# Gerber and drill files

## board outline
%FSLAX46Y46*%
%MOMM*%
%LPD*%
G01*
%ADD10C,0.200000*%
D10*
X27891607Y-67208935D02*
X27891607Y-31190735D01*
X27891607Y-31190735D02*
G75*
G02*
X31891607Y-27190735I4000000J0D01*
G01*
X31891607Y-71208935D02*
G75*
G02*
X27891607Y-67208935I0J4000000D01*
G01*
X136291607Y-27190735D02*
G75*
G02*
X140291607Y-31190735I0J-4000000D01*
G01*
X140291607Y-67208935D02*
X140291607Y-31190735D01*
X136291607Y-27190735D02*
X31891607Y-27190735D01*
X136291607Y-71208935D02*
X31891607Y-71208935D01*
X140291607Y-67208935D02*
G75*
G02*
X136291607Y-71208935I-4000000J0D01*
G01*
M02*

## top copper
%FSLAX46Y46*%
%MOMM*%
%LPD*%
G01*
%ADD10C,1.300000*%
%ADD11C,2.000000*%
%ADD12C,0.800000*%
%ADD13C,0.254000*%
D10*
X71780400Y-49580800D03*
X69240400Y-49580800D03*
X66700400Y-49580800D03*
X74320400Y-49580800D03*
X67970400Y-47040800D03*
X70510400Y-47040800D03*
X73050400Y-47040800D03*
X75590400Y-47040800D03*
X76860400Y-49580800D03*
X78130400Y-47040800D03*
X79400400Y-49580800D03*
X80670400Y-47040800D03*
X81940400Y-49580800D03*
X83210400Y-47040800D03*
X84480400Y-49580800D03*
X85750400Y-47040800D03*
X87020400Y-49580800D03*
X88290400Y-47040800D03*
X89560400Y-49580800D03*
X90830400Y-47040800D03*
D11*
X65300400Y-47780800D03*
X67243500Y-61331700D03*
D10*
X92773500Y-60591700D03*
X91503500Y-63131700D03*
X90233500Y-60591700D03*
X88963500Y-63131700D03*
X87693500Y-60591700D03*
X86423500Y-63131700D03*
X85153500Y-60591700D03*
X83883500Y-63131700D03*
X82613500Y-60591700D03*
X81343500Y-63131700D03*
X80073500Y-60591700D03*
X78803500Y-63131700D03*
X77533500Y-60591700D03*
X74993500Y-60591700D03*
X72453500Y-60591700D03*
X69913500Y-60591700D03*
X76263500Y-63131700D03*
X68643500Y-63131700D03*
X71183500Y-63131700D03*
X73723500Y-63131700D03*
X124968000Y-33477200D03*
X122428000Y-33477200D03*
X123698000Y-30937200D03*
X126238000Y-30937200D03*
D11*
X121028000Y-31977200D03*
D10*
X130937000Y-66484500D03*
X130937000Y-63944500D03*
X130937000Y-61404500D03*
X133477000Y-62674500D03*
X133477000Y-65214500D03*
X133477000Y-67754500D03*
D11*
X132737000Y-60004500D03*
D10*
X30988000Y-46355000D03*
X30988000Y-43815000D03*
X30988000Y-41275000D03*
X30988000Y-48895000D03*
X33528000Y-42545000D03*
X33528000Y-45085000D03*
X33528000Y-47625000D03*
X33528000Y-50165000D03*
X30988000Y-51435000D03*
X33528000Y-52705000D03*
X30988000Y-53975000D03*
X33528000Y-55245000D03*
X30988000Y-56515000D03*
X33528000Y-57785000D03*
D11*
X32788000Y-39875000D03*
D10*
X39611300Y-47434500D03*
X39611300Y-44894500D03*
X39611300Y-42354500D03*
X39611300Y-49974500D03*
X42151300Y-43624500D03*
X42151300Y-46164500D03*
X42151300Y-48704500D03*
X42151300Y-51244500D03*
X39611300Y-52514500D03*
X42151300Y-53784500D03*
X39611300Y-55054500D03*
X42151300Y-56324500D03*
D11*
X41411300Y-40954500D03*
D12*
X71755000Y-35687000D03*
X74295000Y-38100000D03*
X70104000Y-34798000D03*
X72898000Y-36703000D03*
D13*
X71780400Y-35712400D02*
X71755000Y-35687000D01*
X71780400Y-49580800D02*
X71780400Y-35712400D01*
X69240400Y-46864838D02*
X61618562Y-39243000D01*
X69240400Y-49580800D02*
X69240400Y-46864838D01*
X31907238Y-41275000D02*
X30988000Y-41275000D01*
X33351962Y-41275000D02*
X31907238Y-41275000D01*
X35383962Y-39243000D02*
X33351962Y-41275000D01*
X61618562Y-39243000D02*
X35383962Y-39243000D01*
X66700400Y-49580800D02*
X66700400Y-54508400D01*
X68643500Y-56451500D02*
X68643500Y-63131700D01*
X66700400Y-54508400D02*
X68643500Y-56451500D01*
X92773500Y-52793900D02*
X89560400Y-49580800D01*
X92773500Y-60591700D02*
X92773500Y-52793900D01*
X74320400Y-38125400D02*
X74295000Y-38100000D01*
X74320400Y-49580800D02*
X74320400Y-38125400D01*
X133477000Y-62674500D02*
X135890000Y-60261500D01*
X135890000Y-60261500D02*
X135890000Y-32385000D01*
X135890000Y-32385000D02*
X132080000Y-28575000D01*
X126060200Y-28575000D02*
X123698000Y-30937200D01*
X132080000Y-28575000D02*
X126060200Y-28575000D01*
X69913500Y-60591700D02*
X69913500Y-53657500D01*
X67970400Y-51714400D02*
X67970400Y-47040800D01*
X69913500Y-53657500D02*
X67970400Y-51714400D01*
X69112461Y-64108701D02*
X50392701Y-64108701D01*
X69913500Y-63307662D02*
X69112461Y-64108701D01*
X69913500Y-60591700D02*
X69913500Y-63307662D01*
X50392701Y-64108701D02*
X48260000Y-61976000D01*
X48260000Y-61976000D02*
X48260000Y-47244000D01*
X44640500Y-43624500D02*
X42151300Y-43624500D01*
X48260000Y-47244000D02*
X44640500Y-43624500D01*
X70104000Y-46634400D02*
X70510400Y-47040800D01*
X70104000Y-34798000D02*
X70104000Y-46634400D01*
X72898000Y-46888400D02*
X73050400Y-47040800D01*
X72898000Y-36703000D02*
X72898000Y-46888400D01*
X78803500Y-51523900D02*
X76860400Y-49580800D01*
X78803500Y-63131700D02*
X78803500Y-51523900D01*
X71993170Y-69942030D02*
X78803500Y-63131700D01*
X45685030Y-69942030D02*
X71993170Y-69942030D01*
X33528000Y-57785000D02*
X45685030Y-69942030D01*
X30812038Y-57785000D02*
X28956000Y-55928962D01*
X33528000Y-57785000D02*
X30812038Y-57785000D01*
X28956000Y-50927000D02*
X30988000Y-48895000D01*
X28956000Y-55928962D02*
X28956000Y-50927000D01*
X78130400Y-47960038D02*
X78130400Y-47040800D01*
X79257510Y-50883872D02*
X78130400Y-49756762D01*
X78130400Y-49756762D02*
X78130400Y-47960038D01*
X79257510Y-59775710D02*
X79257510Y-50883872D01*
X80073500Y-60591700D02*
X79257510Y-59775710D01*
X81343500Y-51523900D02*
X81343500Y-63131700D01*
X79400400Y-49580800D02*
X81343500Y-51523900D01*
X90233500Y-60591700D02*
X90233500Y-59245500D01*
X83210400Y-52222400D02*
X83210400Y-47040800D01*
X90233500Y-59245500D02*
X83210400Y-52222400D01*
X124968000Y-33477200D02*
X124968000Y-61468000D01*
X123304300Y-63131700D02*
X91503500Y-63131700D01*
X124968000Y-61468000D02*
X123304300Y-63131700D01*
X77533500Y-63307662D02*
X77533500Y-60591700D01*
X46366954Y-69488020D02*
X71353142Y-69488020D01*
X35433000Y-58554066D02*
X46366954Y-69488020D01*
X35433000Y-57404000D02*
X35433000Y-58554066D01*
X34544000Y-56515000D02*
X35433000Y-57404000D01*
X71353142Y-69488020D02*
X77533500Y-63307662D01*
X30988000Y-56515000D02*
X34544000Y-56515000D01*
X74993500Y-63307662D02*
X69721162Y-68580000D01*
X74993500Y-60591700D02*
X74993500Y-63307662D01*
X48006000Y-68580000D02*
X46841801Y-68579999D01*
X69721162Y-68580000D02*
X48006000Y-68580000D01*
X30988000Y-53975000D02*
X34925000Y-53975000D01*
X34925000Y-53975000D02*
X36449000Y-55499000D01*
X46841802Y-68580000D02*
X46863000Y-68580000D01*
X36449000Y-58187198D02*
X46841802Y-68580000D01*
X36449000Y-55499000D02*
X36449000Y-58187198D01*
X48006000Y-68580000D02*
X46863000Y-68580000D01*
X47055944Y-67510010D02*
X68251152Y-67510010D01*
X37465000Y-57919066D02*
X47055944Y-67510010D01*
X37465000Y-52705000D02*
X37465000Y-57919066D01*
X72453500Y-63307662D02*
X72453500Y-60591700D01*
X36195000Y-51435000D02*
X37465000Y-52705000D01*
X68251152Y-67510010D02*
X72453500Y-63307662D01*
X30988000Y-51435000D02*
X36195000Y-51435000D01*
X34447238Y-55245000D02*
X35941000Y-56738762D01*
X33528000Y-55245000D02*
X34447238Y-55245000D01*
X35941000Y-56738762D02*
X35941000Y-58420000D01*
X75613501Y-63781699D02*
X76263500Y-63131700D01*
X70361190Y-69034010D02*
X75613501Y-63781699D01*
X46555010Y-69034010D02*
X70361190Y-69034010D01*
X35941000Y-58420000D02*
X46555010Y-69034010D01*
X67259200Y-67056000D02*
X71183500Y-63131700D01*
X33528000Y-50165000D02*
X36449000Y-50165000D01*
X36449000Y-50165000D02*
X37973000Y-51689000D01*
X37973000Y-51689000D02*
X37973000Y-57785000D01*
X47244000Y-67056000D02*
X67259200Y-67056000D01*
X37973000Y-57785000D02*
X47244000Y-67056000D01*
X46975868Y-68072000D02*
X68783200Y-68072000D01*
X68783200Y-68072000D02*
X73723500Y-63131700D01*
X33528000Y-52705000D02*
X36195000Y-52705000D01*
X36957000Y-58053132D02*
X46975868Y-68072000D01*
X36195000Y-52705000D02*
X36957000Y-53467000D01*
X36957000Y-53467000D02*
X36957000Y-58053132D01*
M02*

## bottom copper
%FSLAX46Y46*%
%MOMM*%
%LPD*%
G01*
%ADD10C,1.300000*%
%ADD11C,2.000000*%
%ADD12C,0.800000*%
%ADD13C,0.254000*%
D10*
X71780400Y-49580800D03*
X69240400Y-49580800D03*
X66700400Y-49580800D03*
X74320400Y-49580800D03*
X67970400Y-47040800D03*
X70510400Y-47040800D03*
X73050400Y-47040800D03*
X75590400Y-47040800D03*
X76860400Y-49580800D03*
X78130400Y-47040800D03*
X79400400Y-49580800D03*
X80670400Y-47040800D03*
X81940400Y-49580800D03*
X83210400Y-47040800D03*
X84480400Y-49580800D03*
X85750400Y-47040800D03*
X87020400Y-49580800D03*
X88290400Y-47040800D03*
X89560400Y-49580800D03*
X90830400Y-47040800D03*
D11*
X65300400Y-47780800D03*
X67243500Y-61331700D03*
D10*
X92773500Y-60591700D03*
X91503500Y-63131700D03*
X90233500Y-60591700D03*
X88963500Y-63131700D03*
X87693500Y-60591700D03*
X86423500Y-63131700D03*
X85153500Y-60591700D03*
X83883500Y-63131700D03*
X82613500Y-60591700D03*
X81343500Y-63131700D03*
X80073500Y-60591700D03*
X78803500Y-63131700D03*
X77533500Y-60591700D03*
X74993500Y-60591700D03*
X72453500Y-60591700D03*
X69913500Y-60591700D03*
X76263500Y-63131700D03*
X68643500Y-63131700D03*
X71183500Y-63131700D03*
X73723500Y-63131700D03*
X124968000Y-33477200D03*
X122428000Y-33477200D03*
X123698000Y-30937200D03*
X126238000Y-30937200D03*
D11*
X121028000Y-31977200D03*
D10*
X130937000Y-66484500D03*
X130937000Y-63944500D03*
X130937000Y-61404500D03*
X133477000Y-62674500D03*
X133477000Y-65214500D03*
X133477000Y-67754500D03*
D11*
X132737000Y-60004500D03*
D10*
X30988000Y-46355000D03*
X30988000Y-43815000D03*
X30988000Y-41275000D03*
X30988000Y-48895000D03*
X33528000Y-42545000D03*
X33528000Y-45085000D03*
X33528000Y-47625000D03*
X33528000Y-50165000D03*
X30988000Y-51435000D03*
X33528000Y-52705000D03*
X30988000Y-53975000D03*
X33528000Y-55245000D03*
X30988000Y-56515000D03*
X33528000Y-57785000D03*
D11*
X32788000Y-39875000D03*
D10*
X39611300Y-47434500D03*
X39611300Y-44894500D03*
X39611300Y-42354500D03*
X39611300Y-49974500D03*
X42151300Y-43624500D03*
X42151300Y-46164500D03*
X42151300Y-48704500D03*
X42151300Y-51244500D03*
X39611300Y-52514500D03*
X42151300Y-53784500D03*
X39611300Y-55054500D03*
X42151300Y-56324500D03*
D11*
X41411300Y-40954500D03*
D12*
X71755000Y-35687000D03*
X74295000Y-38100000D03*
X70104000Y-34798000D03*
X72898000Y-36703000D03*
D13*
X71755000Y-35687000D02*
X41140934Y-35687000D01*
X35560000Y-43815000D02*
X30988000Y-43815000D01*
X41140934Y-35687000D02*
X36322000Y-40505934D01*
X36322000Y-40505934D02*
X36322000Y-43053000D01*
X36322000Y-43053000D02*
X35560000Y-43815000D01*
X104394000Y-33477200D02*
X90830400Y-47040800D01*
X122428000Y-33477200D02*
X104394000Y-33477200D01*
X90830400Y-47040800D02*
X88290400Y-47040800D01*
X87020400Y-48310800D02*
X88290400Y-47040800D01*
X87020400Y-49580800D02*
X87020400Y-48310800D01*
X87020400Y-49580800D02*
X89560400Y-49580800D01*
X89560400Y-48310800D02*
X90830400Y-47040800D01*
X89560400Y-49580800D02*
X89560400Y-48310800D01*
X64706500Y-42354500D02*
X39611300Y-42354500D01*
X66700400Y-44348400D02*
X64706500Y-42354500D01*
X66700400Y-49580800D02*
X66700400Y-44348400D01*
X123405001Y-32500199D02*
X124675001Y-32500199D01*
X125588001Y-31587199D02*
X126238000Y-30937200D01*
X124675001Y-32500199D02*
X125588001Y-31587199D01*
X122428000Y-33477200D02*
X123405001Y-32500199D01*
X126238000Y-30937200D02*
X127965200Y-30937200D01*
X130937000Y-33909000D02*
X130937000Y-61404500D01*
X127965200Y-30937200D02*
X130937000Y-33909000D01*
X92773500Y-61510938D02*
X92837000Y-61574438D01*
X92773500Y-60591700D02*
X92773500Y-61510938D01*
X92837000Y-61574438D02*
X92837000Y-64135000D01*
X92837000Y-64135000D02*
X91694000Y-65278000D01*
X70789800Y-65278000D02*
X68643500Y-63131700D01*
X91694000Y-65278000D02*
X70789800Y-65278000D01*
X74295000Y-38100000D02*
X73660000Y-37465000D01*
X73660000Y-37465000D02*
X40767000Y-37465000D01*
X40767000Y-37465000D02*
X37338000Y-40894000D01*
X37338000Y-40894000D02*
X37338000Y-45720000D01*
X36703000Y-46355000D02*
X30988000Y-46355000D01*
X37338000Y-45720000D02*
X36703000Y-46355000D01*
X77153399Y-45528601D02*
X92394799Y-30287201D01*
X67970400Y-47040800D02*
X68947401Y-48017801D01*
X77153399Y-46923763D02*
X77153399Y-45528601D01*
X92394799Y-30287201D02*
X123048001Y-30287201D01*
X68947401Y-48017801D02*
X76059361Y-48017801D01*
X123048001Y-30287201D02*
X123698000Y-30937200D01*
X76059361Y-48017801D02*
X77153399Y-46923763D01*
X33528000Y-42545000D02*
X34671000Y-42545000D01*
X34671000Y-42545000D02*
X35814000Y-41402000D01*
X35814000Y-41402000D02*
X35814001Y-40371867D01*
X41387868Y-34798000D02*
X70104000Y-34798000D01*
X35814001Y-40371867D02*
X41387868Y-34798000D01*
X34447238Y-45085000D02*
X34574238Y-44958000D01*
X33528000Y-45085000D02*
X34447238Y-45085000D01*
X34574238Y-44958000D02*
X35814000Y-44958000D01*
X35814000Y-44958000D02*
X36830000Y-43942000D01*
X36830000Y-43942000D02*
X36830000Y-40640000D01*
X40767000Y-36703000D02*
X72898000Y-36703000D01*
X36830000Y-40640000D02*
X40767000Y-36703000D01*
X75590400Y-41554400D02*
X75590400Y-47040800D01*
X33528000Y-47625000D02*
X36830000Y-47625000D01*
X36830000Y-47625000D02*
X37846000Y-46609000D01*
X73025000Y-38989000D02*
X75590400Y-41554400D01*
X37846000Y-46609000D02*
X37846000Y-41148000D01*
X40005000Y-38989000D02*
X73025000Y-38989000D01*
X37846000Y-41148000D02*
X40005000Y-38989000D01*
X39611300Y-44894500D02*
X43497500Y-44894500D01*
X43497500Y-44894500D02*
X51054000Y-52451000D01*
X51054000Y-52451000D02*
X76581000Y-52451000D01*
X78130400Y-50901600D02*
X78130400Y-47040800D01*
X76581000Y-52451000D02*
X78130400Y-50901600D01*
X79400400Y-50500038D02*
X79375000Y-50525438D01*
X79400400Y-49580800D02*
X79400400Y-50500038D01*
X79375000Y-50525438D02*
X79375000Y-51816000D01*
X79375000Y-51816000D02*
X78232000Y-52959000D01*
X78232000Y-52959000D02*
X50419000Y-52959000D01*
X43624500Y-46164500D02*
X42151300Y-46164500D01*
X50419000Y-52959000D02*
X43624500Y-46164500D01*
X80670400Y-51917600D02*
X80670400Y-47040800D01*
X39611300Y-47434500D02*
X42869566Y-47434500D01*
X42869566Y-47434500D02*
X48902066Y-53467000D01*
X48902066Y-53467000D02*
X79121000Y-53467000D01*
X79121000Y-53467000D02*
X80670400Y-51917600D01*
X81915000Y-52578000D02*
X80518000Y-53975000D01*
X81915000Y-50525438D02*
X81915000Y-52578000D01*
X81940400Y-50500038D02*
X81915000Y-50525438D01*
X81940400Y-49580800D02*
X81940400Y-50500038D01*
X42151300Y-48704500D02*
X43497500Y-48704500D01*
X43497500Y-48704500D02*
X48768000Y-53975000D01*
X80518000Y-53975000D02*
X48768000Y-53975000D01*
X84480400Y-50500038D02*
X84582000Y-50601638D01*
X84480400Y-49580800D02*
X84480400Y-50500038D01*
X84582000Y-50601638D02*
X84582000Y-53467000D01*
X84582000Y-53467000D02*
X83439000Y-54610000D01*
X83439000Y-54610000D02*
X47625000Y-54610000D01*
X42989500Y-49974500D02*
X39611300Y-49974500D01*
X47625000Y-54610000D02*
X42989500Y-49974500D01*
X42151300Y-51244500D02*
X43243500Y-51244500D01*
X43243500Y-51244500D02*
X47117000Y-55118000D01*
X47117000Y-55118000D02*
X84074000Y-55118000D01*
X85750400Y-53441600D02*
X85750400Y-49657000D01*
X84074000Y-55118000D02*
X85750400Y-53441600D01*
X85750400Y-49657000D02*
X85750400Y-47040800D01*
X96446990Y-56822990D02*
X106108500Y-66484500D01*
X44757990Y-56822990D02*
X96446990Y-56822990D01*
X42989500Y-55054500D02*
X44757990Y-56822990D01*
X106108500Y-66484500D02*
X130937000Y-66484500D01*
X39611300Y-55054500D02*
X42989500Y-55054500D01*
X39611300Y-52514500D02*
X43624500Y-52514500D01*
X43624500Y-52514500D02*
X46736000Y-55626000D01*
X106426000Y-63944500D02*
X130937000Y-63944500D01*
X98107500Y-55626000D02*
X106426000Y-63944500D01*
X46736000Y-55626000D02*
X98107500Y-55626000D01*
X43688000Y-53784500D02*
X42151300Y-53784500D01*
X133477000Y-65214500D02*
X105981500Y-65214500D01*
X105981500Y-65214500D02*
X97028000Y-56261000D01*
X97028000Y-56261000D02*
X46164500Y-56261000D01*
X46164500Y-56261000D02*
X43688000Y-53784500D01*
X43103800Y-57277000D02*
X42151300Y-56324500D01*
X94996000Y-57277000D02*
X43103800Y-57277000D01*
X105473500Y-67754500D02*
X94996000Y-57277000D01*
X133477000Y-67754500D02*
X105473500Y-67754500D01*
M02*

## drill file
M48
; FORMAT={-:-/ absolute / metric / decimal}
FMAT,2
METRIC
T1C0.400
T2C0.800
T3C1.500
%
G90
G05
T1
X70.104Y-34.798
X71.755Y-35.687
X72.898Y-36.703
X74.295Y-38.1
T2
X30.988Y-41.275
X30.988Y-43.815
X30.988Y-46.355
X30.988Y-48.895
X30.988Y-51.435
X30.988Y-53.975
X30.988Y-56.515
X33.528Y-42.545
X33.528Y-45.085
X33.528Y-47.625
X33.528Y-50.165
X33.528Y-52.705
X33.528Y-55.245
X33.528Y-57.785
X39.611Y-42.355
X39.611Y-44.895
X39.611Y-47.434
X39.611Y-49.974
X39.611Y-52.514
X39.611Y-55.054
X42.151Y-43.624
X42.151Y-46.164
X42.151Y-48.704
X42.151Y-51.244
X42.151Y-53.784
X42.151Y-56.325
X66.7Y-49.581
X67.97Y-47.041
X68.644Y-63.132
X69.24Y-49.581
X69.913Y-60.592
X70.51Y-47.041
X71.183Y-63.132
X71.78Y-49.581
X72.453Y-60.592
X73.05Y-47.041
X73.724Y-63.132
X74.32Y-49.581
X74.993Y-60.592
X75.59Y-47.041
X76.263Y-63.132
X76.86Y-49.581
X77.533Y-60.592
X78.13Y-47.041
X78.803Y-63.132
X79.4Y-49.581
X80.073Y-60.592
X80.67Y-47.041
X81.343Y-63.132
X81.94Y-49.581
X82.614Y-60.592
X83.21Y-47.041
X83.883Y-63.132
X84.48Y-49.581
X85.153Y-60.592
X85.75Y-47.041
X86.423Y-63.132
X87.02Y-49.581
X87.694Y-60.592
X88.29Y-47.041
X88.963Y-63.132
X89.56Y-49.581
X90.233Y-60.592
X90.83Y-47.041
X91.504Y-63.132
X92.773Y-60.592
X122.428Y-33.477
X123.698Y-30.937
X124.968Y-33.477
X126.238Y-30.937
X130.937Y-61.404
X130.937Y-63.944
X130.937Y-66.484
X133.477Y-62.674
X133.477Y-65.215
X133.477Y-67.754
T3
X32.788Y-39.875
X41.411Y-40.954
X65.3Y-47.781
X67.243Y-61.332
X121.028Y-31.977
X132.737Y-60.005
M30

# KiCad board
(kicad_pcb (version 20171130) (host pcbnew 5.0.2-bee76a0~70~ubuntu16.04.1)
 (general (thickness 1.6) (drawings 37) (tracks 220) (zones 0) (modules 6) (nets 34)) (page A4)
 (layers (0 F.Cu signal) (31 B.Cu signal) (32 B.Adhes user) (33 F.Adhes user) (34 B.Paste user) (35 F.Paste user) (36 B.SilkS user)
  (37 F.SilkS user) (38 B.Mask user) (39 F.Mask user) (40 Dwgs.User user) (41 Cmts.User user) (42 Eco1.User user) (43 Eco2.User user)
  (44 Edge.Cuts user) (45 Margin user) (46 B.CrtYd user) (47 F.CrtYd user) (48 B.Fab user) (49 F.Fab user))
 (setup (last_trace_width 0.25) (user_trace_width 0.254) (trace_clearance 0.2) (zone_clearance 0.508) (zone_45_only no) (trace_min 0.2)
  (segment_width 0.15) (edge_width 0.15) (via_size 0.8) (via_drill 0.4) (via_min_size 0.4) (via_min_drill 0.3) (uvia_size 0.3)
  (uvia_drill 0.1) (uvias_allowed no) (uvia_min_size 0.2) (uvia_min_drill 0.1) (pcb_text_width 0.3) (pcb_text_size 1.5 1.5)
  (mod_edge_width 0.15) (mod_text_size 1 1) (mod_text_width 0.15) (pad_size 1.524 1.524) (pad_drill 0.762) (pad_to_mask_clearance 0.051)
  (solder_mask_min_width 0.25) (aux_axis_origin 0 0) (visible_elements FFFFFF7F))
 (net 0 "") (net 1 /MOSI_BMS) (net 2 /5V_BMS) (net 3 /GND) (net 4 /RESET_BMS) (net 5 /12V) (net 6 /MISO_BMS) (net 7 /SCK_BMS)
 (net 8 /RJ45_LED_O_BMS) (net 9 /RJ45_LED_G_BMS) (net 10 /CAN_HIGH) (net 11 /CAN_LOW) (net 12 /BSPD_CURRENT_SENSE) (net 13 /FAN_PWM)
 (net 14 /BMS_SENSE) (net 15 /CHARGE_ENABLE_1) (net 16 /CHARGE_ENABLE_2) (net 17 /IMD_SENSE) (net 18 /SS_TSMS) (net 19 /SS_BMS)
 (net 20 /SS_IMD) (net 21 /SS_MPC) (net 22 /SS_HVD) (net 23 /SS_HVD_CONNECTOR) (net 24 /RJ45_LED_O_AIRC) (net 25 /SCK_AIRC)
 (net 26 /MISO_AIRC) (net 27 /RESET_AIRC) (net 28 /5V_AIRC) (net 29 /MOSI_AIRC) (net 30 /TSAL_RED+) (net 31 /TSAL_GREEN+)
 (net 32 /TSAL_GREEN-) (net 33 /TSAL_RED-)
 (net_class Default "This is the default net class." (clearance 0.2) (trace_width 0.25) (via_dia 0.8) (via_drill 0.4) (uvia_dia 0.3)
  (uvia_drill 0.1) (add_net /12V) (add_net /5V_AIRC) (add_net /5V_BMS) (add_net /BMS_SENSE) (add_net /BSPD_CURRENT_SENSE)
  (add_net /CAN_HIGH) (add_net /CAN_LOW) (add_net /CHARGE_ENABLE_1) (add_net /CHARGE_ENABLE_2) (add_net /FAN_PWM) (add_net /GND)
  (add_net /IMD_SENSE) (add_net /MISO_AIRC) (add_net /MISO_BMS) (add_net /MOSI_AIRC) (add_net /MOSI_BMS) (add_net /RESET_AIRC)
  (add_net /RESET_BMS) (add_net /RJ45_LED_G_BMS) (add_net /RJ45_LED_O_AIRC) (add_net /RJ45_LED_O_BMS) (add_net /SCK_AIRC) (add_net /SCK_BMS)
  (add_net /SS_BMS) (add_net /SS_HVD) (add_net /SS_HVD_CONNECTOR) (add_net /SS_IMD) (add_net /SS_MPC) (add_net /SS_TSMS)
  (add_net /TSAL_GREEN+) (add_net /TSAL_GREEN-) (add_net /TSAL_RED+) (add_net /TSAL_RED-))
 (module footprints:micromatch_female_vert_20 (layer F.Cu) (at 71.7804 49.5808 90)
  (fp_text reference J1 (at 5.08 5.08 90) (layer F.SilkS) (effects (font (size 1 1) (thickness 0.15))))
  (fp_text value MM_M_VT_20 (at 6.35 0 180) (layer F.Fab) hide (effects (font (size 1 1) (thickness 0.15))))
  (pad 5 thru_hole circle (at 0 0 90) (size 1.3 1.3) (drill 0.8) (layers *.Cu *.Mask) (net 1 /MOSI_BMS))
  (pad 3 thru_hole circle (at 0 -2.54 90) (size 1.3 1.3) (drill 0.8) (layers *.Cu *.Mask) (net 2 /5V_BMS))
  (pad 1 thru_hole circle (at 0 -5.08 90) (size 1.3 1.3) (drill 0.8) (layers *.Cu *.Mask) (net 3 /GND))
  (pad 7 thru_hole circle (at 0 2.54 90) (size 1.3 1.3) (drill 0.8) (layers *.Cu *.Mask) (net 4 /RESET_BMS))
  (pad 2 thru_hole circle (at 2.54 -3.81 90) (size 1.3 1.3) (drill 0.8) (layers *.Cu *.Mask) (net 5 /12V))
  (pad 4 thru_hole circle (at 2.54 -1.27 90) (size 1.3 1.3) (drill 0.8) (layers *.Cu *.Mask) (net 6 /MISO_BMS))
  (pad 6 thru_hole circle (at 2.54 1.27 90) (size 1.3 1.3) (drill 0.8) (layers *.Cu *.Mask) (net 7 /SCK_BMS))
  (pad 8 thru_hole circle (at 2.54 3.81 90) (size 1.3 1.3) (drill 0.8) (layers *.Cu *.Mask) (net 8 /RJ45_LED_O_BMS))
  (pad 9 thru_hole circle (at 0 5.08 90) (size 1.3 1.3) (drill 0.8) (layers *.Cu *.Mask) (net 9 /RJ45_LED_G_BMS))
  (pad 10 thru_hole circle (at 2.54 6.35 90) (size 1.3 1.3) (drill 0.8) (layers *.Cu *.Mask) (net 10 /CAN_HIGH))
  (pad 11 thru_hole circle (at 0 7.62 90) (size 1.3 1.3) (drill 0.8) (layers *.Cu *.Mask) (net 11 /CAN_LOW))
  (pad 12 thru_hole circle (at 2.54 8.89 90) (size 1.3 1.3) (drill 0.8) (layers *.Cu *.Mask) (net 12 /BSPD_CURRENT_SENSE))
  (pad 13 thru_hole circle (at 0 10.16 90) (size 1.3 1.3) (drill 0.8) (layers *.Cu *.Mask) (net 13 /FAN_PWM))
  (pad 14 thru_hole circle (at 2.54 11.43 90) (size 1.3 1.3) (drill 0.8) (layers *.Cu *.Mask) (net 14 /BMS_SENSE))
  (pad 15 thru_hole circle (at 0 12.7 90) (size 1.3 1.3) (drill 0.8) (layers *.Cu *.Mask) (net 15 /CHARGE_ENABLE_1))
  (pad 16 thru_hole circle (at 2.54 13.97 90) (size 1.3 1.3) (drill 0.8) (layers *.Cu *.Mask) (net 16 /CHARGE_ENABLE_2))
  (pad 17 thru_hole circle (at 0 15.24 90) (size 1.3 1.3) (drill 0.8) (layers *.Cu *.Mask) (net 3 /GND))
  (pad 18 thru_hole circle (at 2.54 16.51 90) (size 1.3 1.3) (drill 0.8) (layers *.Cu *.Mask) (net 3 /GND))
  (pad 19 thru_hole circle (at 0 17.78 90) (size 1.3 1.3) (drill 0.8) (layers *.Cu *.Mask) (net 3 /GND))
  (pad 20 thru_hole circle (at 2.54 19.05 90) (size 1.3 1.3) (drill 0.8) (layers *.Cu *.Mask) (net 3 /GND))
  (pad 21 thru_hole circle (at 1.8 -6.48 90) (size 2 2) (drill 1.5) (layers *.Cu *.Mask)))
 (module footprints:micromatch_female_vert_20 (layer F.Cu) (at 73.7235 63.1317 90)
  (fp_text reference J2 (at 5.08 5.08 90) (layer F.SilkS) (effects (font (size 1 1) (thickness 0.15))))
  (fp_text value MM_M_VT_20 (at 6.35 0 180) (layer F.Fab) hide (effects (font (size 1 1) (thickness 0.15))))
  (pad 21 thru_hole circle (at 1.8 -6.48 90) (size 2 2) (drill 1.5) (layers *.Cu *.Mask))
  (pad 20 thru_hole circle (at 2.54 19.05 90) (size 1.3 1.3) (drill 0.8) (layers *.Cu *.Mask) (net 3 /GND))
  (pad 19 thru_hole circle (at 0 17.78 90) (size 1.3 1.3) (drill 0.8) (layers *.Cu *.Mask) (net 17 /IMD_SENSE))
  (pad 18 thru_hole circle (at 2.54 16.51 90) (size 1.3 1.3) (drill 0.8) (layers *.Cu *.Mask) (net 14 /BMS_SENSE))
  (pad 17 thru_hole circle (at 0 15.24 90) (size 1.3 1.3) (drill 0.8) (layers *.Cu *.Mask) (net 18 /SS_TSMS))
  (pad 16 thru_hole circle (at 2.54 13.97 90) (size 1.3 1.3) (drill 0.8) (layers *.Cu *.Mask) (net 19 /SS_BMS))
  (pad 15 thru_hole circle (at 0 12.7 90) (size 1.3 1.3) (drill 0.8) (layers *.Cu *.Mask) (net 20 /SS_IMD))
  (pad 14 thru_hole circle (at 2.54 11.43 90) (size 1.3 1.3) (drill 0.8) (layers *.Cu *.Mask) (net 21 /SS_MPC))
  (pad 13 thru_hole circle (at 0 10.16 90) (size 1.3 1.3) (drill 0.8) (layers *.Cu *.Mask) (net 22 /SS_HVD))
  (pad 12 thru_hole circle (at 2.54 8.89 90) (size 1.3 1.3) (drill 0.8) (layers *.Cu *.Mask) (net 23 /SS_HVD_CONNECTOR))
  (pad 11 thru_hole circle (at 0 7.62 90) (size 1.3 1.3) (drill 0.8) (layers *.Cu *.Mask) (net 11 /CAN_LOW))
  (pad 10 thru_hole circle (at 2.54 6.35 90) (size 1.3 1.3) (drill 0.8) (layers *.Cu *.Mask) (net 10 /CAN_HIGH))
  (pad 9 thru_hole circle (at 0 5.08 90) (size 1.3 1.3) (drill 0.8) (layers *.Cu *.Mask) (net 9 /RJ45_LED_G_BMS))
  (pad 8 thru_hole circle (at 2.54 3.81 90) (size 1.3 1.3) (drill 0.8) (layers *.Cu *.Mask) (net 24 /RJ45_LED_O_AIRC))
  (pad 6 thru_hole circle (at 2.54 1.27 90) (size 1.3 1.3) (drill 0.8) (layers *.Cu *.Mask) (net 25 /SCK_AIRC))
  (pad 4 thru_hole circle (at 2.54 -1.27 90) (size 1.3 1.3) (drill 0.8) (layers *.Cu *.Mask) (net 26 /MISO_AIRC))
  (pad 2 thru_hole circle (at 2.54 -3.81 90) (size 1.3 1.3) (drill 0.8) (layers *.Cu *.Mask) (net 5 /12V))
  (pad 7 thru_hole circle (at 0 2.54 90) (size 1.3 1.3) (drill 0.8) (layers *.Cu *.Mask) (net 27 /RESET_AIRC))
  (pad 1 thru_hole circle (at 0 -5.08 90) (size 1.3 1.3) (drill 0.8) (layers *.Cu *.Mask) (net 3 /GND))
  (pad 3 thru_hole circle (at 0 -2.54 90) (size 1.3 1.3) (drill 0.8) (layers *.Cu *.Mask) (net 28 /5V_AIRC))
  (pad 5 thru_hole circle (at 0 0 90) (size 1.3 1.3) (drill 0.8) (layers *.Cu *.Mask) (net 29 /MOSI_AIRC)))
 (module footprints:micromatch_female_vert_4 (layer F.Cu) (at 127.508 33.4772 90)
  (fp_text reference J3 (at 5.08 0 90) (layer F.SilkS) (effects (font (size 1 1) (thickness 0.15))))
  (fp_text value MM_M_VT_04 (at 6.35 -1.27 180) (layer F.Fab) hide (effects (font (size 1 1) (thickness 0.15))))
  (pad 3 thru_hole circle (at 0 -2.54 90) (size 1.3 1.3) (drill 0.8) (layers *.Cu *.Mask) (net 17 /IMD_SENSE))
  (pad 1 thru_hole circle (at 0 -5.08 90) (size 1.3 1.3) (drill 0.8) (layers *.Cu *.Mask) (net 3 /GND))
  (pad 2 thru_hole circle (at 2.54 -3.81 90) (size 1.3 1.3) (drill 0.8) (layers *.Cu *.Mask) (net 5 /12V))
  (pad 4 thru_hole circle (at 2.54 -1.27 90) (size 1.3 1.3) (drill 0.8) (layers *.Cu *.Mask) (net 3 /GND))
  (pad 5 thru_hole circle (at 1.5 -6.48 90) (size 2 2) (drill 1.5) (layers *.Cu *.Mask)))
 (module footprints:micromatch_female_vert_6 (layer F.Cu) (at 130.937 66.4845)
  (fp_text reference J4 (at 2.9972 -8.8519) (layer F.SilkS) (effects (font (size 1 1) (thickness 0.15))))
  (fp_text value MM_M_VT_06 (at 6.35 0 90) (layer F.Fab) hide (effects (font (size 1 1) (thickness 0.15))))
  (pad 5 thru_hole circle (at 0 0) (size 1.3 1.3) (drill 0.8) (layers *.Cu *.Mask) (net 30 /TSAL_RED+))
  (pad 3 thru_hole circle (at 0 -2.54) (size 1.3 1.3) (drill 0.8) (layers *.Cu *.Mask) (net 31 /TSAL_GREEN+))
  (pad 1 thru_hole circle (at 0 -5.08) (size 1.3 1.3) (drill 0.8) (layers *.Cu *.Mask) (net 3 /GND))
  (pad 2 thru_hole circle (at 2.54 -3.81) (size 1.3 1.3) (drill 0.8) (layers *.Cu *.Mask) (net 5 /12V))
  (pad 4 thru_hole circle (at 2.54 -1.27) (size 1.3 1.3) (drill 0.8) (layers *.Cu *.Mask) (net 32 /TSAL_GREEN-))
  (pad 6 thru_hole circle (at 2.54 1.27) (size 1.3 1.3) (drill 0.8) (layers *.Cu *.Mask) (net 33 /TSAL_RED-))
  (pad 7 thru_hole circle (at 1.8 -6.48) (size 2 2) (drill 1.5) (layers *.Cu *.Mask)))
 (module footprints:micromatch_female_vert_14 (layer F.Cu) (at 30.988 46.355)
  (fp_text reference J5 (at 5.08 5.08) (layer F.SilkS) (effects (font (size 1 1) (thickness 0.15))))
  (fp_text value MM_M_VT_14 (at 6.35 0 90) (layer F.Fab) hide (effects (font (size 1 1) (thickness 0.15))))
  (pad 5 thru_hole circle (at 0 0) (size 1.3 1.3) (drill 0.8) (layers *.Cu *.Mask) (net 4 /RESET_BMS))
  (pad 3 thru_hole circle (at 0 -2.54) (size 1.3 1.3) (drill 0.8) (layers *.Cu *.Mask) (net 1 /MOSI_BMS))
  (pad 1 thru_hole circle (at 0 -5.08) (size 1.3 1.3) (drill 0.8) (layers *.Cu *.Mask) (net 2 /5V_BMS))
  (pad 7 thru_hole circle (at 0 2.54) (size 1.3 1.3) (drill 0.8) (layers *.Cu *.Mask) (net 9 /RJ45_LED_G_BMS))
  (pad 2 thru_hole circle (at 2.54 -3.81) (size 1.3 1.3) (drill 0.8) (layers *.Cu *.Mask) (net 6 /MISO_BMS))
  (pad 4 thru_hole circle (at 2.54 -1.27) (size 1.3 1.3) (drill 0.8) (layers *.Cu *.Mask) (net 7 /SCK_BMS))
  (pad 6 thru_hole circle (at 2.54 1.27) (size 1.3 1.3) (drill 0.8) (layers *.Cu *.Mask) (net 8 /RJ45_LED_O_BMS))
  (pad 8 thru_hole circle (at 2.54 3.81) (size 1.3 1.3) (drill 0.8) (layers *.Cu *.Mask) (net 28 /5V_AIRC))
  (pad 9 thru_hole circle (at 0 5.08) (size 1.3 1.3) (drill 0.8) (layers *.Cu *.Mask) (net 26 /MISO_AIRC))
  (pad 10 thru_hole circle (at 2.54 6.35) (size 1.3 1.3) (drill 0.8) (layers *.Cu *.Mask) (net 29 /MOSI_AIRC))
  (pad 11 thru_hole circle (at 0 7.62) (size 1.3 1.3) (drill 0.8) (layers *.Cu *.Mask) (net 25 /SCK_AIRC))
  (pad 12 thru_hole circle (at 2.54 8.89) (size 1.3 1.3) (drill 0.8) (layers *.Cu *.Mask) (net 27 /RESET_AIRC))
  (pad 13 thru_hole circle (at 0 10.16) (size 1.3 1.3) (drill 0.8) (layers *.Cu *.Mask) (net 24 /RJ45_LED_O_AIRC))
  (pad 14 thru_hole circle (at 2.54 11.43) (size 1.3 1.3) (drill 0.8) (layers *.Cu *.Mask) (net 9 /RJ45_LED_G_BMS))
  (pad 15 thru_hole circle (at 1.8 -6.48) (size 2 2) (drill 1.5) (layers *.Cu *.Mask)))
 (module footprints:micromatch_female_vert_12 (layer F.Cu) (at 39.6113 47.4345)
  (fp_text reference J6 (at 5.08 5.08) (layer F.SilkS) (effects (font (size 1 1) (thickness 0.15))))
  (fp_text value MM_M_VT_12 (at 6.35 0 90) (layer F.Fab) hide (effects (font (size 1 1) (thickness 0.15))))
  (pad 5 thru_hole circle (at 0 0) (size 1.3 1.3) (drill 0.8) (layers *.Cu *.Mask) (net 12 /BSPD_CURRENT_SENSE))
  (pad 3 thru_hole circle (at 0 -2.54) (size 1.3 1.3) (drill 0.8) (layers *.Cu *.Mask) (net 10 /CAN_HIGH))
  (pad 1 thru_hole circle (at 0 -5.08) (size 1.3 1.3) (drill 0.8) (layers *.Cu *.Mask) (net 3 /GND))
  (pad 7 thru_hole circle (at 0 2.54) (size 1.3 1.3) (drill 0.8) (layers *.Cu *.Mask) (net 15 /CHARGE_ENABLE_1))
  (pad 2 thru_hole circle (at 2.54 -3.81) (size 1.3 1.3) (drill 0.8) (layers *.Cu *.Mask) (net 5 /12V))
  (pad 4 thru_hole circle (at 2.54 -1.27) (size 1.3 1.3) (drill 0.8) (layers *.Cu *.Mask) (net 11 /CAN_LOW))
  (pad 6 thru_hole circle (at 2.54 1.27) (size 1.3 1.3) (drill 0.8) (layers *.Cu *.Mask) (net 13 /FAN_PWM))
  (pad 8 thru_hole circle (at 2.54 3.81) (size 1.3 1.3) (drill 0.8) (layers *.Cu *.Mask) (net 16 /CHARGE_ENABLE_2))
  (pad 9 thru_hole circle (at 0 5.08) (size 1.3 1.3) (drill 0.8) (layers *.Cu *.Mask) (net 31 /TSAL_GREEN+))
  (pad 10 thru_hole circle (at 2.54 6.35) (size 1.3 1.3) (drill 0.8) (layers *.Cu *.Mask) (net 32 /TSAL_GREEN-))
  (pad 11 thru_hole circle (at 0 7.62) (size 1.3 1.3) (drill 0.8) (layers *.Cu *.Mask) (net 30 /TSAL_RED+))
  (pad 12 thru_hole circle (at 2.54 8.89) (size 1.3 1.3) (drill 0.8) (layers *.Cu *.Mask) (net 33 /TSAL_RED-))
  (pad 13 thru_hole circle (at 1.8 -6.48) (size 2 2) (drill 1.5) (layers *.Cu *.Mask)))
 (gr_line (start 27.891607 67.208935) (end 27.891607 31.190735) (layer Edge.Cuts) (width 0.2))
 (gr_arc (start 31.891607 31.190735) (end 31.891607 27.190735) (angle -90) (layer Edge.Cuts) (width 0.2))
 (gr_arc (start 31.891607 67.208935) (end 27.891607 67.208935) (angle -90) (layer Edge.Cuts) (width 0.2))
 (gr_arc (start 136.291607 31.190735) (end 140.291607 31.190735) (angle -90) (layer Edge.Cuts) (width 0.2))
 (gr_line (start 140.291607 67.208935) (end 140.291607 31.190735) (layer Edge.Cuts) (width 0.2))
 (gr_line (start 136.291607 27.190735) (end 31.891607 27.190735) (layer Edge.Cuts) (width 0.2))
 (gr_line (start 136.291607 71.208935) (end 31.891607 71.208935) (layer Edge.Cuts) (width 0.2))
 (gr_arc (start 136.291607 67.208935) (end 136.291607 71.208935) (angle -90) (layer Edge.Cuts) (width 0.2))
 (via (at 71.755 35.687) (size 0.8) (drill 0.4) (layers F.Cu B.Cu) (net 1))
 (segment (start 71.7804 35.7124) (end 71.755 35.687) (width 0.254) (layer F.Cu) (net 1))
 (segment (start 71.7804 49.5808) (end 71.7804 35.7124) (width 0.254) (layer F.Cu) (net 1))
 (segment (start 71.755 35.687) (end 41.140934 35.687) (width 0.254) (layer B.Cu) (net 1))
 (segment (start 35.56 43.815) (end 30.988 43.815) (width 0.254) (layer B.Cu) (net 1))
 (segment (start 41.140934 35.687) (end 36.322 40.505934) (width 0.254) (layer B.Cu) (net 1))
 (segment (start 36.322 40.505934) (end 36.322 43.053) (width 0.254) (layer B.Cu) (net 1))
 (segment (start 36.322 43.053) (end 35.56 43.815) (width 0.254) (layer B.Cu) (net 1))
 (segment (start 69.2404 46.864838) (end 61.618562 39.243) (width 0.254) (layer F.Cu) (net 2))
 (segment (start 69.2404 49.5808) (end 69.2404 46.864838) (width 0.254) (layer F.Cu) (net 2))
 (segment (start 31.907238 41.275) (end 30.988 41.275) (width 0.254) (layer F.Cu) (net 2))
 (segment (start 33.351962 41.275) (end 31.907238 41.275) (width 0.254) (layer F.Cu) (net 2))
 (segment (start 35.383962 39.243) (end 33.351962 41.275) (width 0.254) (layer F.Cu) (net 2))
 (segment (start 61.618562 39.243) (end 35.383962 39.243) (width 0.254) (layer F.Cu) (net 2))
 (segment (start 104.394 33.4772) (end 90.8304 47.0408) (width 0.254) (layer B.Cu) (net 3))
 (segment (start 122.428 33.4772) (end 104.394 33.4772) (width 0.254) (layer B.Cu) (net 3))
 (segment (start 90.8304 47.0408) (end 88.2904 47.0408) (width 0.254) (layer B.Cu) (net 3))
 (segment (start 87.0204 48.3108) (end 88.2904 47.0408) (width 0.254) (layer B.Cu) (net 3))
 (segment (start 87.0204 49.5808) (end 87.0204 48.3108) (width 0.254) (layer B.Cu) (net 3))
 (segment (start 87.0204 49.5808) (end 89.5604 49.5808) (width 0.254) (layer B.Cu) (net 3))
 (segment (start 89.5604 48.3108) (end 90.8304 47.0408) (width 0.254) (layer B.Cu) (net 3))
 (segment (start 89.5604 49.5808) (end 89.5604 48.3108) (width 0.254) (layer B.Cu) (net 3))
 (segment (start 64.7065 42.3545) (end 39.6113 42.3545) (width 0.254) (layer B.Cu) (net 3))
 (segment (start 66.7004 44.3484) (end 64.7065 42.3545) (width 0.254) (layer B.Cu) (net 3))
 (segment (start 66.7004 49.5808) (end 66.7004 44.3484) (width 0.254) (layer B.Cu) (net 3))
 (segment (start 123.405001 32.500199) (end 124.675001 32.500199) (width 0.254) (layer B.Cu) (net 3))
 (segment (start 125.588001 31.587199) (end 126.238 30.9372) (width 0.254) (layer B.Cu) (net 3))
 (segment (start 124.675001 32.500199) (end 125.588001 31.587199) (width 0.254) (layer B.Cu) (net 3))
 (segment (start 122.428 33.4772) (end 123.405001 32.500199) (width 0.254) (layer B.Cu) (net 3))
 (segment (start 126.238 30.9372) (end 127.9652 30.9372) (width 0.254) (layer B.Cu) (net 3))
 (segment (start 130.937 33.909) (end 130.937 61.4045) (width 0.254) (layer B.Cu) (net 3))
 (segment (start 127.9652 30.9372) (end 130.937 33.909) (width 0.254) (layer B.Cu) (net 3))
 (segment (start 66.7004 49.5808) (end 66.7004 54.5084) (width 0.254) (layer F.Cu) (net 3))
 (segment (start 68.6435 56.4515) (end 68.6435 63.1317) (width 0.254) (layer F.Cu) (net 3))
 (segment (start 66.7004 54.5084) (end 68.6435 56.4515) (width 0.254) (layer F.Cu) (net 3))
 (segment (start 92.7735 52.7939) (end 89.5604 49.5808) (width 0.254) (layer F.Cu) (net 3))
 (segment (start 92.7735 60.5917) (end 92.7735 52.7939) (width 0.254) (layer F.Cu) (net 3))
 (segment (start 92.7735 61.510938) (end 92.837 61.574438) (width 0.254) (layer B.Cu) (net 3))
 (segment (start 92.7735 60.5917) (end 92.7735 61.510938) (width 0.254) (layer B.Cu) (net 3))
 (segment (start 92.837 61.574438) (end 92.837 64.135) (width 0.254) (layer B.Cu) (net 3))
 (segment (start 92.837 64.135) (end 91.694 65.278) (width 0.254) (layer B.Cu) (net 3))
 (segment (start 70.7898 65.278) (end 68.6435 63.1317) (width 0.254) (layer B.Cu) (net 3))
 (segment (start 91.694 65.278) (end 70.7898 65.278) (width 0.254) (layer B.Cu) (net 3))
 (via (at 74.295 38.1) (size 0.8) (drill 0.4) (layers F.Cu B.Cu) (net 4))
 (segment (start 74.3204 38.1254) (end 74.295 38.1) (width 0.254) (layer F.Cu) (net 4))
 (segment (start 74.3204 49.5808) (end 74.3204 38.1254) (width 0.254) (layer F.Cu) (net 4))
 (segment (start 74.295 38.1) (end 73.66 37.465) (width 0.254) (layer B.Cu) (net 4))
 (segment (start 73.66 37.465) (end 40.767 37.465) (width 0.254) (layer B.Cu) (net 4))
 (segment (start 40.767 37.465) (end 37.338 40.894) (width 0.254) (layer B.Cu) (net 4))
 (segment (start 37.338 40.894) (end 37.338 45.72) (width 0.254) (layer B.Cu) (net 4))
 (segment (start 36.703 46.355) (end 30.988 46.355) (width 0.254) (layer B.Cu) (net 4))
 (segment (start 37.338 45.72) (end 36.703 46.355) (width 0.254) (layer B.Cu) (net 4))
 (segment (start 133.477 62.6745) (end 135.89 60.2615) (width 0.254) (layer F.Cu) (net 5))
 (segment (start 135.89 60.2615) (end 135.89 32.385) (width 0.254) (layer F.Cu) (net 5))
 (segment (start 135.89 32.385) (end 132.08 28.575) (width 0.254) (layer F.Cu) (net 5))
 (segment (start 126.0602 28.575) (end 123.698 30.9372) (width 0.254) (layer F.Cu) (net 5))
 (segment (start 132.08 28.575) (end 126.0602 28.575) (width 0.254) (layer F.Cu) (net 5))
 (segment (start 69.9135 60.5917) (end 69.9135 53.6575) (width 0.254) (layer F.Cu) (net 5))
 (segment (start 67.9704 51.7144) (end 67.9704 47.0408) (width 0.254) (layer F.Cu) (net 5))
 (segment (start 69.9135 53.6575) (end 67.9704 51.7144) (width 0.254) (layer F.Cu) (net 5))
 (segment (start 69.112461 64.108701) (end 50.392701 64.108701) (width 0.254) (layer F.Cu) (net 5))
 (segment (start 69.9135 63.307662) (end 69.112461 64.108701) (width 0.254) (layer F.Cu) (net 5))
 (segment (start 69.9135 60.5917) (end 69.9135 63.307662) (width 0.254) (layer F.Cu) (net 5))
 (segment (start 50.392701 64.108701) (end 48.26 61.976) (width 0.254) (layer F.Cu) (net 5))
 (segment (start 48.26 61.976) (end 48.26 47.244) (width 0.254) (layer F.Cu) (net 5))
 (segment (start 44.6405 43.6245) (end 42.1513 43.6245) (width 0.254) (layer F.Cu) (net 5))
 (segment (start 48.26 47.244) (end 44.6405 43.6245) (width 0.254) (layer F.Cu) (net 5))
 (segment (start 77.153399 45.528601) (end 92.394799 30.287201) (width 0.254) (layer B.Cu) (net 5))
 (segment (start 67.9704 47.0408) (end 68.947401 48.017801) (width 0.254) (layer B.Cu) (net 5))
 (segment (start 77.153399 46.923763) (end 77.153399 45.528601) (width 0.254) (layer B.Cu) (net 5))
 (segment (start 92.394799 30.287201) (end 123.048001 30.287201) (width 0.254) (layer B.Cu) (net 5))
 (segment (start 68.947401 48.017801) (end 76.059361 48.017801) (width 0.254) (layer B.Cu) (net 5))
 (segment (start 123.048001 30.287201) (end 123.698 30.9372) (width 0.254) (layer B.Cu) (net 5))
 (segment (start 76.059361 48.017801) (end 77.153399 46.923763) (width 0.254) (layer B.Cu) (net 5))
 (segment (start 33.528 42.545) (end 34.671 42.545) (width 0.254) (layer B.Cu) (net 6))
 (segment (start 34.671 42.545) (end 35.814 41.402) (width 0.254) (layer B.Cu) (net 6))
 (segment (start 35.814 41.402) (end 35.814001 40.371867) (width 0.254) (layer B.Cu) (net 6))
 (via (at 70.104 34.798) (size 0.8) (drill 0.4) (layers F.Cu B.Cu) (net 6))
 (segment (start 41.387868 34.798) (end 70.104 34.798) (width 0.254) (layer B.Cu) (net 6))
 (segment (start 35.814001 40.371867) (end 41.387868 34.798) (width 0.254) (layer B.Cu) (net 6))
 (segment (start 70.104 46.6344) (end 70.5104 47.0408) (width 0.254) (layer F.Cu) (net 6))
 (segment (start 70.104 34.798) (end 70.104 46.6344) (width 0.254) (layer F.Cu) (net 6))
 (segment (start 34.447238 45.085) (end 34.574238 44.958) (width 0.254) (layer B.Cu) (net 7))
 (segment (start 33.528 45.085) (end 34.447238 45.085) (width 0.254) (layer B.Cu) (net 7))
 (segment (start 34.574238 44.958) (end 35.814 44.958) (width 0.254) (layer B.Cu) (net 7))
 (segment (start 35.814 44.958) (end 36.83 43.942) (width 0.254) (layer B.Cu) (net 7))
 (segment (start 36.83 43.942) (end 36.83 40.64) (width 0.254) (layer B.Cu) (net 7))
 (via (at 72.898 36.703) (size 0.8) (drill 0.4) (layers F.Cu B.Cu) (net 7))
 (segment (start 40.767 36.703) (end 72.898 36.703) (width 0.254) (layer B.Cu) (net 7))
 (segment (start 36.83 40.64) (end 40.767 36.703) (width 0.254) (layer B.Cu) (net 7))
 (segment (start 72.898 46.8884) (end 73.0504 47.0408) (width 0.254) (layer F.Cu) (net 7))
 (segment (start 72.898 36.703) (end 72.898 46.8884) (width 0.254) (layer F.Cu) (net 7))
 (segment (start 75.5904 41.5544) (end 75.5904 47.0408) (width 0.254) (layer B.Cu) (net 8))
 (segment (start 33.528 47.625) (end 36.83 47.625) (width 0.254) (layer B.Cu) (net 8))
 (segment (start 36.83 47.625) (end 37.846 46.609) (width 0.254) (layer B.Cu) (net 8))
 (segment (start 73.025 38.989) (end 75.5904 41.5544) (width 0.254) (layer B.Cu) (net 8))
 (segment (start 37.846 46.609) (end 37.846 41.148) (width 0.254) (layer B.Cu) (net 8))
 (segment (start 40.005 38.989) (end 73.025 38.989) (width 0.254) (layer B.Cu) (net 8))
 (segment (start 37.846 41.148) (end 40.005 38.989) (width 0.254) (layer B.Cu) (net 8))
 (segment (start 78.8035 51.5239) (end 76.8604 49.5808) (width 0.254) (layer F.Cu) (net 9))
 (segment (start 78.8035 63.1317) (end 78.8035 51.5239) (width 0.254) (layer F.Cu) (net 9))
 (segment (start 71.99317 69.94203) (end 78.8035 63.1317) (width 0.254) (layer F.Cu) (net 9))
 (segment (start 45.68503 69.94203) (end 71.99317 69.94203) (width 0.254) (layer F.Cu) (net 9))
 (segment (start 33.528 57.785) (end 45.68503 69.94203) (width 0.254) (layer F.Cu) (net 9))
 (segment (start 30.812038 57.785) (end 28.956 55.928962) (width 0.254) (layer F.Cu) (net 9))
 (segment (start 33.528 57.785) (end 30.812038 57.785) (width 0.254) (layer F.Cu) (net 9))
 (segment (start 28.956 50.927) (end 30.988 48.895) (width 0.254) (layer F.Cu) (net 9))
 (segment (start 28.956 55.928962) (end 28.956 50.927) (width 0.254) (layer F.Cu) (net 9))
 (segment (start 78.1304 47.960038) (end 78.1304 47.0408) (width 0.254) (layer F.Cu) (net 10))
 (segment (start 79.25751 50.883872) (end 78.1304 49.756762) (width 0.254) (layer F.Cu) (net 10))
 (segment (start 78.1304 49.756762) (end 78.1304 47.960038) (width 0.254) (layer F.Cu) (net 10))
 (segment (start 79.25751 59.77571) (end 79.25751 50.883872) (width 0.254) (layer F.Cu) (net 10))
 (segment (start 80.0735 60.5917) (end 79.25751 59.77571) (width 0.254) (layer F.Cu) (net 10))
 (segment (start 39.6113 44.8945) (end 43.4975 44.8945) (width 0.254) (layer B.Cu) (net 10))
 (segment (start 43.4975 44.8945) (end 51.054 52.451) (width 0.254) (layer B.Cu) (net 10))
 (segment (start 51.054 52.451) (end 76.581 52.451) (width 0.254) (layer B.Cu) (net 10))
 (segment (start 78.1304 50.9016) (end 78.1304 47.0408) (width 0.254) (layer B.Cu) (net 10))
 (segment (start 76.581 52.451) (end 78.1304 50.9016) (width 0.254) (layer B.Cu) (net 10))
 (segment (start 81.3435 51.5239) (end 81.3435 63.1317) (width 0.254) (layer F.Cu) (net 11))
 (segment (start 79.4004 49.5808) (end 81.3435 51.5239) (width 0.254) (layer F.Cu) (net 11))
 (segment (start 79.4004 50.500038) (end 79.375 50.525438) (width 0.254) (layer B.Cu) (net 11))
 (segment (start 79.4004 49.5808) (end 79.4004 50.500038) (width 0.254) (layer B.Cu) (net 11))
 (segment (start 79.375 50.525438) (end 79.375 51.816) (width 0.254) (layer B.Cu) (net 11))
 (segment (start 79.375 51.816) (end 78.232 52.959) (width 0.254) (layer B.Cu) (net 11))
 (segment (start 78.232 52.959) (end 50.419 52.959) (width 0.254) (layer B.Cu) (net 11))
 (segment (start 43.6245 46.1645) (end 42.1513 46.1645) (width 0.254) (layer B.Cu) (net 11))
 (segment (start 50.419 52.959) (end 43.6245 46.1645) (width 0.254) (layer B.Cu) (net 11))
 (segment (start 80.6704 51.9176) (end 80.6704 47.0408) (width 0.254) (layer B.Cu) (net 12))
 (segment (start 39.6113 47.4345) (end 42.869566 47.4345) (width 0.254) (layer B.Cu) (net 12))
 (segment (start 42.869566 47.4345) (end 48.902066 53.467) (width 0.254) (layer B.Cu) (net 12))
 (segment (start 48.902066 53.467) (end 79.121 53.467) (width 0.254) (layer B.Cu) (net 12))
 (segment (start 79.121 53.467) (end 80.6704 51.9176) (width 0.254) (layer B.Cu) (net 12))
 (segment (start 81.915 52.578) (end 80.518 53.975) (width 0.254) (layer B.Cu) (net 13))
 (segment (start 81.915 50.525438) (end 81.915 52.578) (width 0.254) (layer B.Cu) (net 13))
 (segment (start 81.9404 50.500038) (end 81.915 50.525438) (width 0.254) (layer B.Cu) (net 13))
 (segment (start 81.9404 49.5808) (end 81.9404 50.500038) (width 0.254) (layer B.Cu) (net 13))
 (segment (start 42.1513 48.7045) (end 43.4975 48.7045) (width 0.254) (layer B.Cu) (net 13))
 (segment (start 43.4975 48.7045) (end 48.768 53.975) (width 0.254) (layer B.Cu) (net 13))
 (segment (start 80.518 53.975) (end 48.768 53.975) (width 0.254) (layer B.Cu) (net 13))
 (segment (start 90.2335 60.5917) (end 90.2335 59.2455) (width 0.254) (layer F.Cu) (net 14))
 (segment (start 83.2104 52.2224) (end 83.2104 47.0408) (width 0.254) (layer F.Cu) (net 14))
 (segment (start 90.2335 59.2455) (end 83.2104 52.2224) (width 0.254) (layer F.Cu) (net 14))
 (segment (start 84.4804 50.500038) (end 84.582 50.601638) (width 0.254) (layer B.Cu) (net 15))
 (segment (start 84.4804 49.5808) (end 84.4804 50.500038) (width 0.254) (layer B.Cu) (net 15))
 (segment (start 84.582 50.601638) (end 84.582 53.467) (width 0.254) (layer B.Cu) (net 15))
 (segment (start 84.582 53.467) (end 83.439 54.61) (width 0.254) (layer B.Cu) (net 15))
 (segment (start 83.439 54.61) (end 47.625 54.61) (width 0.254) (layer B.Cu) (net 15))
 (segment (start 42.9895 49.9745) (end 39.6113 49.9745) (width 0.254) (layer B.Cu) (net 15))
 (segment (start 47.625 54.61) (end 42.9895 49.9745) (width 0.254) (layer B.Cu) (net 15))
 (segment (start 42.1513 51.2445) (end 43.2435 51.2445) (width 0.254) (layer B.Cu) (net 16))
 (segment (start 43.2435 51.2445) (end 47.117 55.118) (width 0.254) (layer B.Cu) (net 16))
 (segment (start 47.117 55.118) (end 84.074 55.118) (width 0.254) (layer B.Cu) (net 16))
 (segment (start 85.7504 53.4416) (end 85.7504 49.657) (width 0.254) (layer B.Cu) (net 16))
 (segment (start 84.074 55.118) (end 85.7504 53.4416) (width 0.254) (layer B.Cu) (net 16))
 (segment (start 85.7504 49.657) (end 85.7504 47.0408) (width 0.254) (layer B.Cu) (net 16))
 (segment (start 124.968 33.4772) (end 124.968 61.468) (width 0.254) (layer F.Cu) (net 17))
 (segment (start 123.3043 63.1317) (end 91.5035 63.1317) (width 0.254) (layer F.Cu) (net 17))
 (segment (start 124.968 61.468) (end 123.3043 63.1317) (width 0.254) (layer F.Cu) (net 17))
 (segment (start 77.5335 63.307662) (end 77.5335 60.5917) (width 0.254) (layer F.Cu) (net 24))
 (segment (start 46.366954 69.48802) (end 71.353142 69.48802) (width 0.254) (layer F.Cu) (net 24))
 (segment (start 35.433 58.554066) (end 46.366954 69.48802) (width 0.254) (layer F.Cu) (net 24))
 (segment (start 35.433 57.404) (end 35.433 58.554066) (width 0.254) (layer F.Cu) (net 24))
 (segment (start 34.544 56.515) (end 35.433 57.404) (width 0.254) (layer F.Cu) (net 24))
 (segment (start 71.353142 69.48802) (end 77.5335 63.307662) (width 0.254) (layer F.Cu) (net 24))
 (segment (start 30.988 56.515) (end 34.544 56.515) (width 0.254) (layer F.Cu) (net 24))
 (segment (start 74.9935 63.307662) (end 69.721162 68.58) (width 0.254) (layer F.Cu) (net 25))
 (segment (start 74.9935 60.5917) (end 74.9935 63.307662) (width 0.254) (layer F.Cu) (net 25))
 (segment (start 48.006 68.58) (end 46.841801 68.579999) (width 0.254) (layer F.Cu) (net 25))
 (segment (start 69.721162 68.58) (end 48.006 68.58) (width 0.254) (layer F.Cu) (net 25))
 (segment (start 30.988 53.975) (end 34.925 53.975) (width 0.254) (layer F.Cu) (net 25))
 (segment (start 34.925 53.975) (end 36.449 55.499) (width 0.254) (layer F.Cu) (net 25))
 (segment (start 46.841802 68.58) (end 46.863 68.58) (width 0.254) (layer F.Cu) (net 25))
 (segment (start 36.449 58.187198) (end 46.841802 68.58) (width 0.254) (layer F.Cu) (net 25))
 (segment (start 36.449 55.499) (end 36.449 58.187198) (width 0.254) (layer F.Cu) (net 25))
 (segment (start 48.006 68.58) (end 46.863 68.58) (width 0.254) (layer F.Cu) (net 25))
 (segment (start 47.055944 67.51001) (end 68.251152 67.51001) (width 0.254) (layer F.Cu) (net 26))
 (segment (start 37.465 57.919066) (end 47.055944 67.51001) (width 0.254) (layer F.Cu) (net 26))
 (segment (start 37.465 52.705) (end 37.465 57.919066) (width 0.254) (layer F.Cu) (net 26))
 (segment (start 72.4535 63.307662) (end 72.4535 60.5917) (width 0.254) (layer F.Cu) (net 26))
 (segment (start 36.195 51.435) (end 37.465 52.705) (width 0.254) (layer F.Cu) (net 26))
 (segment (start 68.251152 67.51001) (end 72.4535 63.307662) (width 0.254) (layer F.Cu) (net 26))
 (segment (start 30.988 51.435) (end 36.195 51.435) (width 0.254) (layer F.Cu) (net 26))
 (segment (start 34.447238 55.245) (end 35.941 56.738762) (width 0.254) (layer F.Cu) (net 27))
 (segment (start 33.528 55.245) (end 34.447238 55.245) (width 0.254) (layer F.Cu) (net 27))
 (segment (start 35.941 56.738762) (end 35.941 58.42) (width 0.254) (layer F.Cu) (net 27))
 (segment (start 75.613501 63.781699) (end 76.2635 63.1317) (width 0.254) (layer F.Cu) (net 27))
 (segment (start 70.36119 69.03401) (end 75.613501 63.781699) (width 0.254) (layer F.Cu) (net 27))
 (segment (start 46.55501 69.03401) (end 70.36119 69.03401) (width 0.254) (layer F.Cu) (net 27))
 (segment (start 35.941 58.42) (end 46.55501 69.03401) (width 0.254) (layer F.Cu) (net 27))
 (segment (start 67.2592 67.056) (end 71.1835 63.1317) (width 0.254) (layer F.Cu) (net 28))
 (segment (start 33.528 50.165) (end 36.449 50.165) (width 0.254) (layer F.Cu) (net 28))
 (segment (start 36.449 50.165) (end 37.973 51.689) (width 0.254) (layer F.Cu) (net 28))
 (segment (start 37.973 51.689) (end 37.973 57.785) (width 0.254) (layer F.Cu) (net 28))
 (segment (start 47.244 67.056) (end 67.2592 67.056) (width 0.254) (layer F.Cu) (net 28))
 (segment (start 37.973 57.785) (end 47.244 67.056) (width 0.254) (layer F.Cu) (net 28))
 (segment (start 46.975868 68.072) (end 68.7832 68.072) (width 0.254) (layer F.Cu) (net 29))
 (segment (start 68.7832 68.072) (end 73.7235 63.1317) (width 0.254) (layer F.Cu) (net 29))
 (segment (start 33.528 52.705) (end 36.195 52.705) (width 0.254) (layer F.Cu) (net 29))
 (segment (start 36.957 58.053132) (end 46.975868 68.072) (width 0.254) (layer F.Cu) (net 29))
 (segment (start 36.195 52.705) (end 36.957 53.467) (width 0.254) (layer F.Cu) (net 29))
 (segment (start 36.957 53.467) (end 36.957 58.053132) (width 0.254) (layer F.Cu) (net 29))
 (segment (start 96.44699 56.82299) (end 106.1085 66.4845) (width 0.254) (layer B.Cu) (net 30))
 (segment (start 44.75799 56.82299) (end 96.44699 56.82299) (width 0.254) (layer B.Cu) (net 30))
 (segment (start 42.9895 55.0545) (end 44.75799 56.82299) (width 0.254) (layer B.Cu) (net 30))
 (segment (start 106.1085 66.4845) (end 130.937 66.4845) (width 0.254) (layer B.Cu) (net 30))
 (segment (start 39.6113 55.0545) (end 42.9895 55.0545) (width 0.254) (layer B.Cu) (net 30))
 (segment (start 39.6113 52.5145) (end 43.6245 52.5145) (width 0.254) (layer B.Cu) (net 31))
 (segment (start 43.6245 52.5145) (end 46.736 55.626) (width 0.254) (layer B.Cu) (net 31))
 (segment (start 106.426 63.9445) (end 130.937 63.9445) (width 0.254) (layer B.Cu) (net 31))
 (segment (start 98.1075 55.626) (end 106.426 63.9445) (width 0.254) (layer B.Cu) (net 31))
 (segment (start 46.736 55.626) (end 98.1075 55.626) (width 0.254) (layer B.Cu) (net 31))
 (segment (start 43.688 53.7845) (end 42.1513 53.7845) (width 0.254) (layer B.Cu) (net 32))
 (segment (start 133.477 65.2145) (end 105.9815 65.2145) (width 0.254) (layer B.Cu) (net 32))
 (segment (start 105.9815 65.2145) (end 97.028 56.261) (width 0.254) (layer B.Cu) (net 32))
 (segment (start 97.028 56.261) (end 46.1645 56.261) (width 0.254) (layer B.Cu) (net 32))
 (segment (start 46.1645 56.261) (end 43.688 53.7845) (width 0.254) (layer B.Cu) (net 32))
 (segment (start 43.1038 57.277) (end 42.1513 56.3245) (width 0.254) (layer B.Cu) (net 33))
 (segment (start 94.996 57.277) (end 43.1038 57.277) (width 0.254) (layer B.Cu) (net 33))
 (segment (start 105.4735 67.7545) (end 94.996 57.277) (width 0.254) (layer B.Cu) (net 33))
 (segment (start 133.477 67.7545) (end 105.4735 67.7545) (width 0.254) (layer B.Cu) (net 33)))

